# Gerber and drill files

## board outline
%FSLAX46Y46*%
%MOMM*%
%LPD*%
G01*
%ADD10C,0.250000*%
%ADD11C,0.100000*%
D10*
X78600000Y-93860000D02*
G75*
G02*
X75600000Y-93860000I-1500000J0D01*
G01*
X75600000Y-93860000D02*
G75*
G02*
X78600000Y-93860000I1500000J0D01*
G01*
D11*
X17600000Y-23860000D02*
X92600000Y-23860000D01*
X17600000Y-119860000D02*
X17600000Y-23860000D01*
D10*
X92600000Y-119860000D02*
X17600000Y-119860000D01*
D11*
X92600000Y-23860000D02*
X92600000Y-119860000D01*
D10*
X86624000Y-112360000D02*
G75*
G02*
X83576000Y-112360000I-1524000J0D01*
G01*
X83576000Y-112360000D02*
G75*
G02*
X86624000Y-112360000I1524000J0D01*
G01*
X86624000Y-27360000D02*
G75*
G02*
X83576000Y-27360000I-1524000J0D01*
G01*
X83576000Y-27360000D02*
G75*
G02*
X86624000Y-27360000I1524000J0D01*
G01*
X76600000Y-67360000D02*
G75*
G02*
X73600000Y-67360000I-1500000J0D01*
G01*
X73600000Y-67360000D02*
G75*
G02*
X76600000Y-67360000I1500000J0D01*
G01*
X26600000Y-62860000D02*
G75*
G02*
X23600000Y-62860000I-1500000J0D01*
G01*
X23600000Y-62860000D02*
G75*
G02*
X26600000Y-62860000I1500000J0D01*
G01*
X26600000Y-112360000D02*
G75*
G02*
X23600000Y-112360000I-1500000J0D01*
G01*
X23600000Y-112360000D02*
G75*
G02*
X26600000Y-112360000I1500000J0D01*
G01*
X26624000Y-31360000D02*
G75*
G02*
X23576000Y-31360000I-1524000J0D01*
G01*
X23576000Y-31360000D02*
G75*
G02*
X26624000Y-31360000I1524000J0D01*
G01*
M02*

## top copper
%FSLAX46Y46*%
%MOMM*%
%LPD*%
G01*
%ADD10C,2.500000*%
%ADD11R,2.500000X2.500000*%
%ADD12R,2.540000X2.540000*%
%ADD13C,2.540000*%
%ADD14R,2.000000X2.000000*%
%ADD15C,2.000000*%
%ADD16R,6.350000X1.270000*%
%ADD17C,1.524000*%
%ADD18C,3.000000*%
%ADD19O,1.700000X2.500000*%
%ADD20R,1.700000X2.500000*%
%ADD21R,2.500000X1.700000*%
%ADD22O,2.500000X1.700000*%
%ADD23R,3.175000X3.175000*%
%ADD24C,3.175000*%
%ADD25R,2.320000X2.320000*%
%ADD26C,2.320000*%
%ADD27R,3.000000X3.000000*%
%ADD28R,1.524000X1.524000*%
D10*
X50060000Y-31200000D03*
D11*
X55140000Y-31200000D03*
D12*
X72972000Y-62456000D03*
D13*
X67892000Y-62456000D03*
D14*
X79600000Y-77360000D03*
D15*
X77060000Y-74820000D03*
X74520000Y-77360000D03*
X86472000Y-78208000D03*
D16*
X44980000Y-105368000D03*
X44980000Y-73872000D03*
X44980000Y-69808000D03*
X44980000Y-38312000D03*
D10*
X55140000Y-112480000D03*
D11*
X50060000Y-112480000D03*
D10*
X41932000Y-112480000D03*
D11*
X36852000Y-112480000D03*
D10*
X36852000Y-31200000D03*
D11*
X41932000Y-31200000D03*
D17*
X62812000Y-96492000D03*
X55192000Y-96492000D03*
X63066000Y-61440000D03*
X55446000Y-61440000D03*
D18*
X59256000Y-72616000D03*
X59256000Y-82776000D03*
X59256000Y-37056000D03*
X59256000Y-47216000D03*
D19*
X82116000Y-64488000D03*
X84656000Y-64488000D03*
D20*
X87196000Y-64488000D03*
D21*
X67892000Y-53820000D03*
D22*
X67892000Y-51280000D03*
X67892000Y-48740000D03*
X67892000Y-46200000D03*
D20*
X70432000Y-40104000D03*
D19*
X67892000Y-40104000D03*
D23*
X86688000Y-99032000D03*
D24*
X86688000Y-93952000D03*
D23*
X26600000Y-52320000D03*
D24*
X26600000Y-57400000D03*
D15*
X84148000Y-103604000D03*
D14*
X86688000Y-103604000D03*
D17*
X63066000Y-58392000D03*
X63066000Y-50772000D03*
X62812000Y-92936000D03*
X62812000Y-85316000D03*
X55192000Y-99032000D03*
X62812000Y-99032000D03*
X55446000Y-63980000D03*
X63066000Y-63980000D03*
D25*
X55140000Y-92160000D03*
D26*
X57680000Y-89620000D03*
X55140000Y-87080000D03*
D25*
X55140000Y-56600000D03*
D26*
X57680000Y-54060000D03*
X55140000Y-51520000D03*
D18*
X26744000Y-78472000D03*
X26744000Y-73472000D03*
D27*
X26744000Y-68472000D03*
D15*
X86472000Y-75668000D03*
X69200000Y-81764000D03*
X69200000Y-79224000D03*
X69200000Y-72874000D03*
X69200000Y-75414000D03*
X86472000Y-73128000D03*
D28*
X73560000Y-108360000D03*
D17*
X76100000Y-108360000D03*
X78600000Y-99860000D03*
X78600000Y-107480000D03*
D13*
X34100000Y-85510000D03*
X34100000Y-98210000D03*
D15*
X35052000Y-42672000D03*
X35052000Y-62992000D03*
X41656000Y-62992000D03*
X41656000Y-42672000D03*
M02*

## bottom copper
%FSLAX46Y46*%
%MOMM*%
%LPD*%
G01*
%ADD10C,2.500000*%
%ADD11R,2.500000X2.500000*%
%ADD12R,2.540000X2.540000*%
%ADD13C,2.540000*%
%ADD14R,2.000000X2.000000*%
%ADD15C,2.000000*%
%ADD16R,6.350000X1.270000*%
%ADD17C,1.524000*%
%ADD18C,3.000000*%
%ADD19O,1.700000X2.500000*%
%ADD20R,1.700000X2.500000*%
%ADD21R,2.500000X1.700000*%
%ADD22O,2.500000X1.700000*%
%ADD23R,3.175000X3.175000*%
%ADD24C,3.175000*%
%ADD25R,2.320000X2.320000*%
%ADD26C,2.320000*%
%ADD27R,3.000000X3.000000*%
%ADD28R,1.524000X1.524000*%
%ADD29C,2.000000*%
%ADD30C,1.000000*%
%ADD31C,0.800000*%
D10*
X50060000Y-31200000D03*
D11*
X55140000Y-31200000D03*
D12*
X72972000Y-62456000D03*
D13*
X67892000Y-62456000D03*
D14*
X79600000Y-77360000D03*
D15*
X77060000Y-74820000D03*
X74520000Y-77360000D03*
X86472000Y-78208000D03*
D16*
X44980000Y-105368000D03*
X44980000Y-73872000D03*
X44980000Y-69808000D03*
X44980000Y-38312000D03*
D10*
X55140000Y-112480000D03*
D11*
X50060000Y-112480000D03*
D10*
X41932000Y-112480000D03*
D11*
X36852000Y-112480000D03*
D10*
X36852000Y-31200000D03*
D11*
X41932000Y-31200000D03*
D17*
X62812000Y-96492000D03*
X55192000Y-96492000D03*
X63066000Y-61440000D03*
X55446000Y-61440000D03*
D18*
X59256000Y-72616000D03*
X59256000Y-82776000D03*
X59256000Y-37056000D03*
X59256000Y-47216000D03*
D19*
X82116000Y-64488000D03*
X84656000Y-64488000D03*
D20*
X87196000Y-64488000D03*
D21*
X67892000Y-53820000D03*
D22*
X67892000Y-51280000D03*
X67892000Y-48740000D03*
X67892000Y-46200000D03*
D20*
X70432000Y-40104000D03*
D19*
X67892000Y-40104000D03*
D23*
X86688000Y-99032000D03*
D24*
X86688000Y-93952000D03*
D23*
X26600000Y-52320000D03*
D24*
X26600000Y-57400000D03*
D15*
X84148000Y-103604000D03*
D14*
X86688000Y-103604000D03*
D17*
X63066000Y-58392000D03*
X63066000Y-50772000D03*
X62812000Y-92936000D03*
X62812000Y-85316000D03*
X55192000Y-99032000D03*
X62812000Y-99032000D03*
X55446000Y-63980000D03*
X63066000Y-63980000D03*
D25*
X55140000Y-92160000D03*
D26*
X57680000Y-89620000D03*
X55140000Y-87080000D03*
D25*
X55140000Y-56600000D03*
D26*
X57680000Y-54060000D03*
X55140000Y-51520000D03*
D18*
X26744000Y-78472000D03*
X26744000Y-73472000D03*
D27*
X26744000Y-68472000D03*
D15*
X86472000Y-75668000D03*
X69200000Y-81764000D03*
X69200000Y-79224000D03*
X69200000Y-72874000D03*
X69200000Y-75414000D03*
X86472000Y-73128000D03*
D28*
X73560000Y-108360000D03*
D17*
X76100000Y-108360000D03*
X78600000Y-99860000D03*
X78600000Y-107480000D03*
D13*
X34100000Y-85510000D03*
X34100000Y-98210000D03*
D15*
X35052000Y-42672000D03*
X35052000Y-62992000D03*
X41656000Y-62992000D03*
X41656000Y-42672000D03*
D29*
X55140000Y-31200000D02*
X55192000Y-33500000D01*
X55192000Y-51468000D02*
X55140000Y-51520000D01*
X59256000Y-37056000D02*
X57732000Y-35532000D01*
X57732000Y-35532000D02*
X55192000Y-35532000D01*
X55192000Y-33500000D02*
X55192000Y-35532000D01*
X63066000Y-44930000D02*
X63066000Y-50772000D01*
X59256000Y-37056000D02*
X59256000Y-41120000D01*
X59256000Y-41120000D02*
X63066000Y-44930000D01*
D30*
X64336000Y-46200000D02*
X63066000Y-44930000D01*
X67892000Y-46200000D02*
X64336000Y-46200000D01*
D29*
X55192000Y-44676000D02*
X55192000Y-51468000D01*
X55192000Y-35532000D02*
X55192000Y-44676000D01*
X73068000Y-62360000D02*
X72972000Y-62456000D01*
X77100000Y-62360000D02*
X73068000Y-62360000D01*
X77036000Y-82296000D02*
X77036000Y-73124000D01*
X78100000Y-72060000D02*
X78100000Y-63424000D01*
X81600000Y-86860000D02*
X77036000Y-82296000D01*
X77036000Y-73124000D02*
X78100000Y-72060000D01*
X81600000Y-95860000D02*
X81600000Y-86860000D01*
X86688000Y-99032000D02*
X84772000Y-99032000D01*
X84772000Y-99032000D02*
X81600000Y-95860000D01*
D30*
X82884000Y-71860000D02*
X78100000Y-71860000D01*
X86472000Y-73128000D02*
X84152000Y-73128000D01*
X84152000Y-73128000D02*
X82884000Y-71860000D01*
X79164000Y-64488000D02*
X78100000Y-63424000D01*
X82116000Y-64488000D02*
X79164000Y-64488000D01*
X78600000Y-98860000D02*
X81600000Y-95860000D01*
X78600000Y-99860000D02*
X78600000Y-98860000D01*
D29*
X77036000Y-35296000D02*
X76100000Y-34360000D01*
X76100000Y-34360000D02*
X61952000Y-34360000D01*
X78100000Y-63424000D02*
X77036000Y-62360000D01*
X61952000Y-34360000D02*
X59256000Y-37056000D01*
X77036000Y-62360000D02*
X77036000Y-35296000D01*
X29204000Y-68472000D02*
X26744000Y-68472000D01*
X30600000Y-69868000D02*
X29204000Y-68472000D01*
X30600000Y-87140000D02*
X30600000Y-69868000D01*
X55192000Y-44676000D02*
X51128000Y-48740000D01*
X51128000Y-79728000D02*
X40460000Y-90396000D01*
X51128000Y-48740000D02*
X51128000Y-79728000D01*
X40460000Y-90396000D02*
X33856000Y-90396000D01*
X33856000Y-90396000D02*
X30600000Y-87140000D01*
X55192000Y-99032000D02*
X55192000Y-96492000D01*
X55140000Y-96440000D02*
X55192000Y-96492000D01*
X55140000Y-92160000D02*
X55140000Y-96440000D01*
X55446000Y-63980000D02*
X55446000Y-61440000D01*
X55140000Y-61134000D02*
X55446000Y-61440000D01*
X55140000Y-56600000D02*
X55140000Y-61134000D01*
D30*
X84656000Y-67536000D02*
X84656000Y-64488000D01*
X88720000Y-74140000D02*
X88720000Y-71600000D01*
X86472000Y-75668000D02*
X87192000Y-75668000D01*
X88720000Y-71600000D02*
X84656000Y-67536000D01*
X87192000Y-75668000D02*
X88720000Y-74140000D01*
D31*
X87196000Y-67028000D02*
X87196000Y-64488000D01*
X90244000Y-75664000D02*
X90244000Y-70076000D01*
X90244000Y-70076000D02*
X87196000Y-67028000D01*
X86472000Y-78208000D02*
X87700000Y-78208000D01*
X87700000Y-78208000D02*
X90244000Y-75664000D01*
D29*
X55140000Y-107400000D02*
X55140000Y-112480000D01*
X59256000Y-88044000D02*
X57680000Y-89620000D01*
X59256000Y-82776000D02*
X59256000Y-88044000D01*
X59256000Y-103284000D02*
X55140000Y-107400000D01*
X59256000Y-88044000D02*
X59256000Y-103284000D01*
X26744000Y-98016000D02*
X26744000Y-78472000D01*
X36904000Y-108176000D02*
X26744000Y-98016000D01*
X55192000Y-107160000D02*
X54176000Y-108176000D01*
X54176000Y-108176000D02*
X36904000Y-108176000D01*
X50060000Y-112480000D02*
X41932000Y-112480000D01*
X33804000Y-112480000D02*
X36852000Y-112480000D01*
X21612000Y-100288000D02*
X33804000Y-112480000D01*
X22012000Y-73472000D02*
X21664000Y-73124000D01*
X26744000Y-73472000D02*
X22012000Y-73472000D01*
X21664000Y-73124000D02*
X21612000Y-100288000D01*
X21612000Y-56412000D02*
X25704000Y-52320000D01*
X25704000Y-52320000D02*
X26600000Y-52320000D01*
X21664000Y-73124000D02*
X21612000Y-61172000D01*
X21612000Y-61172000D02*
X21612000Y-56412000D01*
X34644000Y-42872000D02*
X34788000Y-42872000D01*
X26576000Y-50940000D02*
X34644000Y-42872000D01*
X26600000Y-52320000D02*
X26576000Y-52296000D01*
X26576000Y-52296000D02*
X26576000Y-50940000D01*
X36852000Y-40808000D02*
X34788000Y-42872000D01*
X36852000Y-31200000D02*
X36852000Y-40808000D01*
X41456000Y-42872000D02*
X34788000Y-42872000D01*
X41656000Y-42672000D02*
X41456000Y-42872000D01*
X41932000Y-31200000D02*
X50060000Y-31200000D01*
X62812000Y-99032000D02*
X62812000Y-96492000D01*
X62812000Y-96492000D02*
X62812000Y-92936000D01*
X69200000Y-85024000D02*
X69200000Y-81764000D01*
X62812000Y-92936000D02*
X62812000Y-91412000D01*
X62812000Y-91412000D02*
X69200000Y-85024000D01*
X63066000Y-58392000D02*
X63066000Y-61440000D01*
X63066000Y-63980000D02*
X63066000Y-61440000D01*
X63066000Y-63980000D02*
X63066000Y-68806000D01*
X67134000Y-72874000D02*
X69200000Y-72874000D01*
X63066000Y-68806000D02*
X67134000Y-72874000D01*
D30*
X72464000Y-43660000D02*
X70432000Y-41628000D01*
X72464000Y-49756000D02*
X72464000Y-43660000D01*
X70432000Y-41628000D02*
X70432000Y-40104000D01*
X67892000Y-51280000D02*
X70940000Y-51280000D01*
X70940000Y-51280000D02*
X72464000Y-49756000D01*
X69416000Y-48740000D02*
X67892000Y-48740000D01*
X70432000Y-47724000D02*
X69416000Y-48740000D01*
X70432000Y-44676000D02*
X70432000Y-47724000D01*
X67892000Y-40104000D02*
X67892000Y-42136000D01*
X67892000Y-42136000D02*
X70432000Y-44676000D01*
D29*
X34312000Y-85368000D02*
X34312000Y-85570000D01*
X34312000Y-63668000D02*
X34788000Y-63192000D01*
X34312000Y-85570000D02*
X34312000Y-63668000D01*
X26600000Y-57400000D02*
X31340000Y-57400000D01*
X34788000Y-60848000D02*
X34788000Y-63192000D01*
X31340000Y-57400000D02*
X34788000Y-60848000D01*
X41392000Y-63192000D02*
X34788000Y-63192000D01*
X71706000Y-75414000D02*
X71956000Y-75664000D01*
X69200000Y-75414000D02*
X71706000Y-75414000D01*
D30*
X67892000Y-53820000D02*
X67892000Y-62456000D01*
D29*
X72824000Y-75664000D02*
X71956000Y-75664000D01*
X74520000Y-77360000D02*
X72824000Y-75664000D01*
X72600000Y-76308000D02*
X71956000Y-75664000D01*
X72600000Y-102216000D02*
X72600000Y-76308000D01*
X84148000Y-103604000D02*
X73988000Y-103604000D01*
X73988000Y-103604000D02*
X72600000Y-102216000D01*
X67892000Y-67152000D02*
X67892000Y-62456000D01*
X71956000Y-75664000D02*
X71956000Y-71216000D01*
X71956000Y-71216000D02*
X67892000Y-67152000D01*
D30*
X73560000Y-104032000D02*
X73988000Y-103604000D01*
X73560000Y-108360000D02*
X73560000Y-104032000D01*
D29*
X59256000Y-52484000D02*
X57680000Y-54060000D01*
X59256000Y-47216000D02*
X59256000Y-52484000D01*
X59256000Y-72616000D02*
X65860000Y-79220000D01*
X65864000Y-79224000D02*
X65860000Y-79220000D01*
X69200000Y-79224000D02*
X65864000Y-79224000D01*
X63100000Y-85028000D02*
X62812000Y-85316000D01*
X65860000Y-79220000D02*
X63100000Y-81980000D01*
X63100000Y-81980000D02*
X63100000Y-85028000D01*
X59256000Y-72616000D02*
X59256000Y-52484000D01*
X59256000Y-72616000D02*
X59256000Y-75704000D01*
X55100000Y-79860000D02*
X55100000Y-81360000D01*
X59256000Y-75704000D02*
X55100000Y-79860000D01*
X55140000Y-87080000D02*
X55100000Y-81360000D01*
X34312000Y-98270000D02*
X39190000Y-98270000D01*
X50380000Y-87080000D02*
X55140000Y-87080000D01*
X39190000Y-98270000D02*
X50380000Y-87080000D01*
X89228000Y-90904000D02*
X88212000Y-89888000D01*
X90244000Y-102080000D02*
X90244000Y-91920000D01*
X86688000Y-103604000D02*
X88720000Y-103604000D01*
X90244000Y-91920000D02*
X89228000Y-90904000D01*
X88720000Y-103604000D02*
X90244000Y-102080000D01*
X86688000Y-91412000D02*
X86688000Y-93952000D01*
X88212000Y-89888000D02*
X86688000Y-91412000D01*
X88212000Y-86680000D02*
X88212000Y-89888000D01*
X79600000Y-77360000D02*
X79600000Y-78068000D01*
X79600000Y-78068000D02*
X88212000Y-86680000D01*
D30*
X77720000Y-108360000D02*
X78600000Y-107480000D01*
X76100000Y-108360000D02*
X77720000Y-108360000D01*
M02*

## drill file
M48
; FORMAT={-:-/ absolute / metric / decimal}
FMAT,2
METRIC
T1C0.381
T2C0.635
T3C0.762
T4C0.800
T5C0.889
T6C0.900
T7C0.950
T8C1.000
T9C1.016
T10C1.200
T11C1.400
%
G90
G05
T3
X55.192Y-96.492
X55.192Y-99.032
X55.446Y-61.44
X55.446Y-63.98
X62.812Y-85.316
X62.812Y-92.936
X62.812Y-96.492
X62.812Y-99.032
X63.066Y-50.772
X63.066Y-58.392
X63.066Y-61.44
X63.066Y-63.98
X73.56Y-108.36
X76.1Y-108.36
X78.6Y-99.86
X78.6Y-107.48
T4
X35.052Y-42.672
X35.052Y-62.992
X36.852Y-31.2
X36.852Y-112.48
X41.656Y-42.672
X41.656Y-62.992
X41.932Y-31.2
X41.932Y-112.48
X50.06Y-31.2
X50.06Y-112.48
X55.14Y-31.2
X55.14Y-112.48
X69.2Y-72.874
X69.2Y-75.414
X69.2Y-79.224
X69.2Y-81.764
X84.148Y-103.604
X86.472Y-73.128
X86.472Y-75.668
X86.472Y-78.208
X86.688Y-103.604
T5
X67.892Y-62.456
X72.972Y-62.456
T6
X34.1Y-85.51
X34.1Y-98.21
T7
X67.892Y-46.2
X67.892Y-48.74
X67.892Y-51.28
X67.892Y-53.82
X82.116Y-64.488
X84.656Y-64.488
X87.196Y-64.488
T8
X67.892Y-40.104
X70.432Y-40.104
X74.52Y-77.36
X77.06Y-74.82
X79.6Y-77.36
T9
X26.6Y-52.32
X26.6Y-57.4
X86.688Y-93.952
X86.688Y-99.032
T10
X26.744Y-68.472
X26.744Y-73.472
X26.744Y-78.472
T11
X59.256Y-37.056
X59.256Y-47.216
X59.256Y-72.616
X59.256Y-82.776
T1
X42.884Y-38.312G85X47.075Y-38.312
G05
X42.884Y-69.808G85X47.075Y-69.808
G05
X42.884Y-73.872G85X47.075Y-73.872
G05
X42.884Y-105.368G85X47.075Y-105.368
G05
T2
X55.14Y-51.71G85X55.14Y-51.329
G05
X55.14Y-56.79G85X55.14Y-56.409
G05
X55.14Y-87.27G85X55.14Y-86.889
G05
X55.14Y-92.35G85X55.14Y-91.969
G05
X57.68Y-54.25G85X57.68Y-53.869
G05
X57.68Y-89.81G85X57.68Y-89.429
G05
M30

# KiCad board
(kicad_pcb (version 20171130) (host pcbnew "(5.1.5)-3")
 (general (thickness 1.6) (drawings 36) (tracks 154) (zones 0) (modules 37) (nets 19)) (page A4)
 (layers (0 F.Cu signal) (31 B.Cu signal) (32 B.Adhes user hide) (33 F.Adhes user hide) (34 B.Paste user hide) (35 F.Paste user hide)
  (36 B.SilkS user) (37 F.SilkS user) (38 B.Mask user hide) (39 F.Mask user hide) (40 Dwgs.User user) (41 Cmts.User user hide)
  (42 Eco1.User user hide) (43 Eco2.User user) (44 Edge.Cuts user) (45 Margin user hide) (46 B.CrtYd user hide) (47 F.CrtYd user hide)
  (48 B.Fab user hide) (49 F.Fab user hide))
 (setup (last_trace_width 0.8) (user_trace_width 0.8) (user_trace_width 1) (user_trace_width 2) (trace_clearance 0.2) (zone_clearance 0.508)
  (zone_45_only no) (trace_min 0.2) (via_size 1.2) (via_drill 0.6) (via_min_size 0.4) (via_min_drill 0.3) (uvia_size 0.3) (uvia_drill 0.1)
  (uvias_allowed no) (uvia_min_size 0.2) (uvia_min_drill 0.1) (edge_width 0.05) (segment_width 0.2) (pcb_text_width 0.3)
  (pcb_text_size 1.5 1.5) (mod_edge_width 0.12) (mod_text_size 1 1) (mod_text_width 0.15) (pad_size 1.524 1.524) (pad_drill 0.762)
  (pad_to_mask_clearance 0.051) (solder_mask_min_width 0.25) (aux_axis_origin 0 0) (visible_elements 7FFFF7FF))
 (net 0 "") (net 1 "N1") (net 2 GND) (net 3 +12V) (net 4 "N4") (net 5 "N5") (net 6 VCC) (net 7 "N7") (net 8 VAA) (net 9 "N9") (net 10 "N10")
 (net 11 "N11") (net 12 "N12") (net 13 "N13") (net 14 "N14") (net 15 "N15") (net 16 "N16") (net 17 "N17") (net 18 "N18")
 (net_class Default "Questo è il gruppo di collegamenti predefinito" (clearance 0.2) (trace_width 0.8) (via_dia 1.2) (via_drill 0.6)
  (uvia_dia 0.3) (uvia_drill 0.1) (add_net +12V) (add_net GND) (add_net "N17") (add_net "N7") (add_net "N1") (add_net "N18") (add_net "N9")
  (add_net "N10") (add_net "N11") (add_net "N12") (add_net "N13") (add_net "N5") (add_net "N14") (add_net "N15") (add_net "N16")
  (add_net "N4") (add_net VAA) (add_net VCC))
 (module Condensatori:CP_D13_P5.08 (layer F.Cu) (at 52.6 31.2 180)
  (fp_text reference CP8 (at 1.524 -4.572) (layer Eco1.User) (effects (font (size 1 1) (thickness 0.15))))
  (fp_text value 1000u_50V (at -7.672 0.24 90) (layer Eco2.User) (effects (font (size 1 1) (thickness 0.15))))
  (pad 2 thru_hole circle (at 2.54 0 180) (size 2.5 2.5) (drill 0.8) (layers *.Cu *.Mask) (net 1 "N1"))
  (pad 1 thru_hole rect (at -2.54 0 180) (size 2.5 2.5) (drill 0.8) (layers *.Cu *.Mask) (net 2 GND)))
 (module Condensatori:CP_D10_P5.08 (layer F.Cu) (at 72.972 62.456 180)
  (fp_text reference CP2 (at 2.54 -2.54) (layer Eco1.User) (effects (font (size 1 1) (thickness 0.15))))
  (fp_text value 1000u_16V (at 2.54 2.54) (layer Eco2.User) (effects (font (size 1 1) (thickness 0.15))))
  (pad 1 thru_hole rect (at 0 0 180) (size 2.54 2.54) (drill 0.889) (layers *.Cu *.Mask) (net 2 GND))
  (pad 2 thru_hole circle (at 5.08 0 180) (size 2.54 2.54) (drill 0.889) (layers *.Cu *.Mask) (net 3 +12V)))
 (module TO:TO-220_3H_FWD (layer F.Cu) (at 79.6 77.36 180)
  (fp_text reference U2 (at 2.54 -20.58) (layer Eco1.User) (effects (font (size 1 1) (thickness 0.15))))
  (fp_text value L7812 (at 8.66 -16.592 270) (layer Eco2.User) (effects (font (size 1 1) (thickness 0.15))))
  (pad 1 thru_hole rect (at 0 0 180) (size 2 2) (drill 1) (layers *.Cu *.Mask) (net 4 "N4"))
  (pad 2 thru_hole circle (at 2.54 2.54 180) (size 2 2) (drill 1) (layers *.Cu *.Mask) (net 2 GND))
  (pad 3 thru_hole circle (at 5.08 0 180) (size 2 2) (drill 1) (layers *.Cu *.Mask) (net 3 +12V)))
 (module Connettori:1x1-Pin (layer F.Cu) (at 86.472 78.208 180)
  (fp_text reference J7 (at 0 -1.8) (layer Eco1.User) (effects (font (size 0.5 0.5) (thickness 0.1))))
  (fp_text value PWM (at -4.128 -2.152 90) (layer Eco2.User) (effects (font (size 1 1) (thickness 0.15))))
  (pad 1 thru_hole circle (at 0 0 180) (size 2 2) (drill 0.8) (layers *.Cu *.Mask) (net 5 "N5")))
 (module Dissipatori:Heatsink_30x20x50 (layer F.Cu) (at 32.28 104.86 90)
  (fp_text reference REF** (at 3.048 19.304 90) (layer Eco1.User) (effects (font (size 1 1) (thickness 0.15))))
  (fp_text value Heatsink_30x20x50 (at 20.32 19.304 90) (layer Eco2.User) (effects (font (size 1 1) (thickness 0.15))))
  (pad "" thru_hole rect (at -0.508 12.7 90) (size 1.27 6.35) (drill oval 0.381 4.572) (layers *.Cu *.Mask))
  (pad "" thru_hole rect (at 30.988 12.7 90) (size 1.27 6.35) (drill oval 0.381 4.572) (layers *.Cu *.Mask)))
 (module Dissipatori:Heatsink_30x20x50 (layer F.Cu) (at 32.28 69.3 90)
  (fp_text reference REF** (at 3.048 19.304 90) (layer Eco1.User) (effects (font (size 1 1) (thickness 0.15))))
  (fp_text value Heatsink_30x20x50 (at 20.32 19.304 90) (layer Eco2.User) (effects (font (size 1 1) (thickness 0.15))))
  (pad "" thru_hole rect (at -0.508 12.7 90) (size 1.27 6.35) (drill oval 0.381 4.572) (layers *.Cu *.Mask))
  (pad "" thru_hole rect (at 30.988 12.7 90) (size 1.27 6.35) (drill oval 0.381 4.572) (layers *.Cu *.Mask)))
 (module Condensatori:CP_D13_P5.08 (layer F.Cu) (at 52.6 112.48)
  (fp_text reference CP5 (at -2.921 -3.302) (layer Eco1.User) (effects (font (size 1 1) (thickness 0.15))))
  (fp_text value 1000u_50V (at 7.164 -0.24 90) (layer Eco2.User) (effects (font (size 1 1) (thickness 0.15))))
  (pad 2 thru_hole circle (at 2.54 0) (size 2.5 2.5) (drill 0.8) (layers *.Cu *.Mask) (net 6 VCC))
  (pad 1 thru_hole rect (at -2.54 0) (size 2.5 2.5) (drill 0.8) (layers *.Cu *.Mask) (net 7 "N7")))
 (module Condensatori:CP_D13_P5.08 (layer F.Cu) (at 39.392 112.48)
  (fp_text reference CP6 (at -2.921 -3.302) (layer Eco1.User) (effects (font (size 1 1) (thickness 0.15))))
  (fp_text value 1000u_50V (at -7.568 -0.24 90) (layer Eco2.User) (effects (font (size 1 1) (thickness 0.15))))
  (pad 2 thru_hole circle (at 2.54 0) (size 2.5 2.5) (drill 0.8) (layers *.Cu *.Mask) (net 7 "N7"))
  (pad 1 thru_hole rect (at -2.54 0) (size 2.5 2.5) (drill 0.8) (layers *.Cu *.Mask) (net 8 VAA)))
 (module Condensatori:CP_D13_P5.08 (layer F.Cu) (at 39.392 31.2 180)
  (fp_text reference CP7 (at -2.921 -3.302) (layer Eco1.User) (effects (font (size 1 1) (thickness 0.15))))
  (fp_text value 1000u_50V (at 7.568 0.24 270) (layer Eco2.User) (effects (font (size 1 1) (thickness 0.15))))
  (pad 2 thru_hole circle (at 2.54 0 180) (size 2.5 2.5) (drill 0.8) (layers *.Cu *.Mask) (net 8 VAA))
  (pad 1 thru_hole rect (at -2.54 0 180) (size 2.5 2.5) (drill 0.8) (layers *.Cu *.Mask) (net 1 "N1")))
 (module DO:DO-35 (layer F.Cu) (at 59.002 96.492 180)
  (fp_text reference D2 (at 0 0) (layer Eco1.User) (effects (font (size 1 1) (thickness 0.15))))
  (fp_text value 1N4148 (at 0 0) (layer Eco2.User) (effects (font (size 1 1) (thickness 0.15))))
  (pad 1 thru_hole circle (at -3.81 0 180) (size 1.524 1.524) (drill 0.762) (layers *.Cu *.Mask) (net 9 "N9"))
  (pad 2 thru_hole circle (at 3.81 0 180) (size 1.524 1.524) (drill 0.762) (layers *.Cu *.Mask) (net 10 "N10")))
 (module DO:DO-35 (layer F.Cu) (at 59.256 61.44 180)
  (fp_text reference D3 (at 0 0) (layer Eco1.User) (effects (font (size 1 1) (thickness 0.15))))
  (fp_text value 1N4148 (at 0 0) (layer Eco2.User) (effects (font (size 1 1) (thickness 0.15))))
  (pad 1 thru_hole circle (at -3.81 0 180) (size 1.524 1.524) (drill 0.762) (layers *.Cu *.Mask) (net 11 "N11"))
  (pad 2 thru_hole circle (at 3.81 0 180) (size 1.524 1.524) (drill 0.762) (layers *.Cu *.Mask) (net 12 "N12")))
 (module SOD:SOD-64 (layer F.Cu) (at 59.256 77.696 90)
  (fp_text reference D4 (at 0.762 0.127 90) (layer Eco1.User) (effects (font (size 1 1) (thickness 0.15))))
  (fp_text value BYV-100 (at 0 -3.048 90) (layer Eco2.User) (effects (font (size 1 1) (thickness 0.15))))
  (pad 2 thru_hole circle (at 5.08 0 90) (size 3 3) (drill 1.4) (layers *.Cu *.Mask) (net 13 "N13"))
  (pad 1 thru_hole circle (at -5.08 0 90) (size 3 3) (drill 1.4) (layers *.Cu *.Mask) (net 6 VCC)))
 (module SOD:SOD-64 (layer F.Cu) (at 59.256 42.136 90)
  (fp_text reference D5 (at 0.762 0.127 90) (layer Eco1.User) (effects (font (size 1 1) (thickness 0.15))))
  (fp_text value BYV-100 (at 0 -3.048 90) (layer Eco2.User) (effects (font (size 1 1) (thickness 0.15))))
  (pad 2 thru_hole circle (at 5.08 0 90) (size 3 3) (drill 1.4) (layers *.Cu *.Mask) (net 2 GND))
  (pad 1 thru_hole circle (at -5.08 0 90) (size 3 3) (drill 1.4) (layers *.Cu *.Mask) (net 13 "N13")))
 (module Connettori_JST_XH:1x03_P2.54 (layer F.Cu) (at 87.196 64.488 180)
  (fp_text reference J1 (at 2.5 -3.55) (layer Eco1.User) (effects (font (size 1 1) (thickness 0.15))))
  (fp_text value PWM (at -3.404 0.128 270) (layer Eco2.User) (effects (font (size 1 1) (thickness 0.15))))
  (pad 3 thru_hole oval (at 5.08 0 180) (size 1.7 2.5) (drill 0.95) (layers *.Cu *.Mask) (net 2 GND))
  (pad 2 thru_hole oval (at 2.54 0 180) (size 1.7 2.5) (drill 0.95) (layers *.Cu *.Mask) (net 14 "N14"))
  (pad 1 thru_hole rect (at 0 0 180) (size 1.7 2.5) (drill 0.95) (layers *.Cu *.Mask) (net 5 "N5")))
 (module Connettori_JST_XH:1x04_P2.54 (layer F.Cu) (at 67.892 53.82 90)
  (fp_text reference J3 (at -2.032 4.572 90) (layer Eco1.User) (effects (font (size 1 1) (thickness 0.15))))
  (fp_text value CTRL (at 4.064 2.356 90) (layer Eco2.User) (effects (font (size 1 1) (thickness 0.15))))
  (pad 1 thru_hole rect (at 0 0 90) (size 1.7 2.5) (drill 0.95) (layers *.Cu *.Mask) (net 3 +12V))
  (pad 2 thru_hole oval (at 2.54 0 90) (size 1.7 2.5) (drill 0.95) (layers *.Cu *.Mask) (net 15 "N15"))
  (pad 3 thru_hole oval (at 5.08 0 90) (size 1.7 2.5) (drill 0.95) (layers *.Cu *.Mask) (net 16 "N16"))
  (pad 4 thru_hole oval (at 7.62 0 90) (size 1.7 2.5) (drill 0.95) (layers *.Cu *.Mask) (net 2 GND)))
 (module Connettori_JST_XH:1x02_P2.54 (layer F.Cu) (at 70.432 40.104 180)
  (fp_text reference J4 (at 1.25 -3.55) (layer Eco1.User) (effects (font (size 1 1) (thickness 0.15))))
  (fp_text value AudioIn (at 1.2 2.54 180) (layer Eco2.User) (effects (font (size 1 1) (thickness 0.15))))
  (pad 1 thru_hole rect (at 0 0 180) (size 1.7 2.5) (drill 1) (layers *.Cu *.Mask) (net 15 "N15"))
  (pad 2 thru_hole oval (at 2.54 0 180) (size 1.7 2.5) (drill 1) (layers *.Cu *.Mask) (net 16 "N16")))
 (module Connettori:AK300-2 (layer F.Cu) (at 86.688 96.492 90)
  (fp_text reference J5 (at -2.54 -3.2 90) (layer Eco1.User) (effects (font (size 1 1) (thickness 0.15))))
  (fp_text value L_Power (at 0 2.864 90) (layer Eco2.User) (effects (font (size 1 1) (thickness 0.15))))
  (pad 1 thru_hole rect (at -2.54 0 90) (size 3.175 3.175) (drill 1.016) (layers *.Cu F.Paste F.Mask) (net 2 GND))
  (pad 2 thru_hole circle (at 2.54 0 90) (size 3.175 3.175) (drill 1.016) (layers *.Cu F.Paste F.Mask) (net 4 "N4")))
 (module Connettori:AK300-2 (layer F.Cu) (at 26.6 54.86 270)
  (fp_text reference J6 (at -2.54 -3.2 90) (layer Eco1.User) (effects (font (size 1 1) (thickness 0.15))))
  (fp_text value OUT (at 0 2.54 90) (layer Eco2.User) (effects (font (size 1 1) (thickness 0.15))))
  (pad 1 thru_hole rect (at -2.54 0 270) (size 3.175 3.175) (drill 1.016) (layers *.Cu F.Paste F.Mask) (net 8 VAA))
  (pad 2 thru_hole circle (at 2.54 0 270) (size 3.175 3.175) (drill 1.016) (layers *.Cu F.Paste F.Mask) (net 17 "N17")))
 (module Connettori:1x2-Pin (layer F.Cu) (at 86.688 103.604 270)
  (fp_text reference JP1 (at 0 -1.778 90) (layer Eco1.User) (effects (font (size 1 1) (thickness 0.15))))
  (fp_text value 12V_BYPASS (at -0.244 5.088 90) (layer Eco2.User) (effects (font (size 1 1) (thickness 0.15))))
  (pad 2 thru_hole circle (at 0 2.54 180) (size 2 2) (drill 0.8) (layers *.Cu *.Mask) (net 3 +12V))
  (pad 1 thru_hole rect (at 0 0 180) (size 2 2) (drill 0.8) (layers *.Cu *.Mask) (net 4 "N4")))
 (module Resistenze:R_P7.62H (layer F.Cu) (at 63.066 54.582 270)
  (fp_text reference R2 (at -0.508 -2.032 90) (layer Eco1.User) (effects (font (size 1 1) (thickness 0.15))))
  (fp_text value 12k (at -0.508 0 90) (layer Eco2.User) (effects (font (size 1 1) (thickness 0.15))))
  (pad 2 thru_hole circle (at 3.81 0 270) (size 1.524 1.524) (drill 0.762) (layers *.Cu *.Mask) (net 11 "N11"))
  (pad 1 thru_hole circle (at -3.81 0 270) (size 1.524 1.524) (drill 0.762) (layers *.Cu *.Mask) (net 2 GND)))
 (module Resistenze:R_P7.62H (layer F.Cu) (at 62.812 89.126 270)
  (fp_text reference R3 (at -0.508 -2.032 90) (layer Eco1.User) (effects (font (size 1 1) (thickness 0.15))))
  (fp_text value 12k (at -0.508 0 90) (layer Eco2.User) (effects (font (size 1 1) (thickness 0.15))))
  (pad 2 thru_hole circle (at 3.81 0 270) (size 1.524 1.524) (drill 0.762) (layers *.Cu *.Mask) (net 9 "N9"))
  (pad 1 thru_hole circle (at -3.81 0 270) (size 1.524 1.524) (drill 0.762) (layers *.Cu *.Mask) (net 13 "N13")))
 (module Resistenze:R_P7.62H (layer F.Cu) (at 59.002 99.032 180)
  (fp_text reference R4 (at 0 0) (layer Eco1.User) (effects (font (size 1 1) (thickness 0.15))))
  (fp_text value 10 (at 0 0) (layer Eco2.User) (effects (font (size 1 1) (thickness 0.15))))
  (pad 2 thru_hole circle (at 3.81 0 180) (size 1.524 1.524) (drill 0.762) (layers *.Cu *.Mask) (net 10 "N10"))
  (pad 1 thru_hole circle (at -3.81 0 180) (size 1.524 1.524) (drill 0.762) (layers *.Cu *.Mask) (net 9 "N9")))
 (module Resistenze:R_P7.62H (layer F.Cu) (at 59.256 63.98 180)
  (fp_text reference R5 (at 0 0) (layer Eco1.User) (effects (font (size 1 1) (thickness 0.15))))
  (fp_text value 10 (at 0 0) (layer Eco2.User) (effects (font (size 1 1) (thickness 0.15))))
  (pad 2 thru_hole circle (at 3.81 0 180) (size 1.524 1.524) (drill 0.762) (layers *.Cu *.Mask) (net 12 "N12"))
  (pad 1 thru_hole circle (at -3.81 0 180) (size 1.524 1.524) (drill 0.762) (layers *.Cu *.Mask) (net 11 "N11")))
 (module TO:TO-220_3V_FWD (layer F.Cu) (at 55.14 89.62 90)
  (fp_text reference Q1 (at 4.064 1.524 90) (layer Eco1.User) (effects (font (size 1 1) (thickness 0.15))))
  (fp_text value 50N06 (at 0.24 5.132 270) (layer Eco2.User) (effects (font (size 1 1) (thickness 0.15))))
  (pad 1 thru_hole rect (at -2.54 0 90) (size 2.32 2.32) (drill oval 1.016 0.635) (layers *.Cu *.Mask) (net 10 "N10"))
  (pad 2 thru_hole circle (at 0 2.54 90) (size 2.32 2.32) (drill oval 1.016 0.635) (layers *.Cu *.Mask) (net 6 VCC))
  (pad 3 thru_hole circle (at 2.54 0 90) (size 2.32 2.32) (drill oval 1.016 0.635) (layers *.Cu *.Mask) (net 13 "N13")))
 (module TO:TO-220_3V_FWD (layer F.Cu) (at 55.14 54.06 90)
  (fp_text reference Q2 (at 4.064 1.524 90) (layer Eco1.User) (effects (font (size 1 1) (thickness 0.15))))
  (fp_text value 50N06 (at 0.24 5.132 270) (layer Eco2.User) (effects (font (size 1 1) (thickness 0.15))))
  (pad 1 thru_hole rect (at -2.54 0 90) (size 2.32 2.32) (drill oval 1.016 0.635) (layers *.Cu *.Mask) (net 12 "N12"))
  (pad 2 thru_hole circle (at 0 2.54 90) (size 2.32 2.32) (drill oval 1.016 0.635) (layers *.Cu *.Mask) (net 13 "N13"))
  (pad 3 thru_hole circle (at 2.54 0 90) (size 2.32 2.32) (drill oval 1.016 0.635) (layers *.Cu *.Mask) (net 2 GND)))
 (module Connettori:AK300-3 (layer F.Cu) (at 26.744 73.552 270)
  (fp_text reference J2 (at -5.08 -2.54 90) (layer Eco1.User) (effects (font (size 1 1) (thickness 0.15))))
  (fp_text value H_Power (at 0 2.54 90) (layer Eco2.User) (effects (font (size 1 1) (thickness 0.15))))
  (pad 3 thru_hole circle (at 4.92 0 270) (size 3 3) (drill 1.2) (layers *.Cu F.Paste F.Mask) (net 6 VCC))
  (pad 2 thru_hole circle (at -0.08 0 270) (size 3 3) (drill 1.2) (layers *.Cu F.Paste F.Mask) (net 8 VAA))
  (pad 1 thru_hole rect (at -5.08 0 270) (size 3 3) (drill 1.2) (layers *.Cu F.Paste F.Mask) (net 2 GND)))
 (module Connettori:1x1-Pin (layer F.Cu) (at 86.472 75.668 180)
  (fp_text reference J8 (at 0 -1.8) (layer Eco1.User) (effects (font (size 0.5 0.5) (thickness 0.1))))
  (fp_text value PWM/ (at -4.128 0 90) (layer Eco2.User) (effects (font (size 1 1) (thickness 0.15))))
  (pad 1 thru_hole circle (at 0 0 180) (size 2 2) (drill 0.8) (layers *.Cu *.Mask) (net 14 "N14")))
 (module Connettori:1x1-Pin (layer F.Cu) (at 69.2 81.764)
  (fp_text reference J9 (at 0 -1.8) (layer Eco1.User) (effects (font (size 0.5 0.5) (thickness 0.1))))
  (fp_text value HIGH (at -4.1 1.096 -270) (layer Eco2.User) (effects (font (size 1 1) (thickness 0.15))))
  (pad 1 thru_hole circle (at 0 0) (size 2 2) (drill 0.8) (layers *.Cu *.Mask) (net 9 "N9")))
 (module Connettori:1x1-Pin (layer F.Cu) (at 69.2 79.224)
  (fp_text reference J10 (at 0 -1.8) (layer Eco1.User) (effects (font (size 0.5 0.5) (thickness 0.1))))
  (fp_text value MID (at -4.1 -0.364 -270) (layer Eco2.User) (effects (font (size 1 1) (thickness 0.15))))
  (pad 1 thru_hole circle (at 0 0) (size 2 2) (drill 0.8) (layers *.Cu *.Mask) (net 13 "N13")))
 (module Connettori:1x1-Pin (layer F.Cu) (at 69.2 72.874)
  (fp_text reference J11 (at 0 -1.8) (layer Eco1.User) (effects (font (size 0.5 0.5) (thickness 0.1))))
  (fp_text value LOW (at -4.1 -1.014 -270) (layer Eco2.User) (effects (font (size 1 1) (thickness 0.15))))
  (pad 1 thru_hole circle (at 0 0) (size 2 2) (drill 0.8) (layers *.Cu *.Mask) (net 11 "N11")))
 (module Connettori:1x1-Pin (layer F.Cu) (at 69.2 75.414)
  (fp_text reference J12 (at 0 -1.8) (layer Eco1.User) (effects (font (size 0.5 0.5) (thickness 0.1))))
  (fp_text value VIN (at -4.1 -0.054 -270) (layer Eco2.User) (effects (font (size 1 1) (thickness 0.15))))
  (pad 1 thru_hole circle (at 0 0) (size 2 2) (drill 0.8) (layers *.Cu *.Mask) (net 3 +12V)))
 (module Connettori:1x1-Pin (layer F.Cu) (at 86.472 73.128 180)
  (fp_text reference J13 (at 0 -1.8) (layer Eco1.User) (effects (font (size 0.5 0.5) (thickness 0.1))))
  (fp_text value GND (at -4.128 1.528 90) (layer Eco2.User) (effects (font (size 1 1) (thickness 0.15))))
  (pad 1 thru_hole circle (at 0 0 180) (size 2 2) (drill 0.8) (layers *.Cu *.Mask) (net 2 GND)))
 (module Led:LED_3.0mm (layer F.Cu) (at 73.56 108.36)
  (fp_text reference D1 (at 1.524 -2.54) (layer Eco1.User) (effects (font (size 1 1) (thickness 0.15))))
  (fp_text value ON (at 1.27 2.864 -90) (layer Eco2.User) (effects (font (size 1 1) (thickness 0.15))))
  (pad 1 thru_hole rect (at 0 0) (size 1.524 1.524) (drill 0.762) (layers *.Cu *.Mask) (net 3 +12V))
  (pad 2 thru_hole circle (at 2.54 0) (size 1.524 1.524) (drill 0.762) (layers *.Cu *.Mask) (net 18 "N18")))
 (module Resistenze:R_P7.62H (layer F.Cu) (at 78.6 103.67 90)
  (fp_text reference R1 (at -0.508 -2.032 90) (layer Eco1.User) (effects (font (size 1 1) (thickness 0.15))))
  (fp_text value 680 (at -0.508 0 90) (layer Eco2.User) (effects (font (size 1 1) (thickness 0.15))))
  (pad 2 thru_hole circle (at 3.81 0 90) (size 1.524 1.524) (drill 0.762) (layers *.Cu *.Mask) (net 2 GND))
  (pad 1 thru_hole circle (at -3.81 0 90) (size 1.524 1.524) (drill 0.762) (layers *.Cu *.Mask) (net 18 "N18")))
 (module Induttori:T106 (layer F.Cu) (at 34.1 91.86 90)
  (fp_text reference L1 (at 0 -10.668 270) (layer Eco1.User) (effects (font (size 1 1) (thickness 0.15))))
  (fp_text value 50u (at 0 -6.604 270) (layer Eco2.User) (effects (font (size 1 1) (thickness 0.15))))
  (pad 2 thru_hole circle (at 6.35 0 90) (size 2.54 2.54) (drill 0.9) (layers *.Cu *.Mask) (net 17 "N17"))
  (pad 1 thru_hole circle (at -6.35 0 90) (size 2.54 2.54) (drill 0.9) (layers *.Cu *.Mask) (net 13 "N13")))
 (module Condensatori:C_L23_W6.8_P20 (layer F.Cu) (at 35.052 42.672 270)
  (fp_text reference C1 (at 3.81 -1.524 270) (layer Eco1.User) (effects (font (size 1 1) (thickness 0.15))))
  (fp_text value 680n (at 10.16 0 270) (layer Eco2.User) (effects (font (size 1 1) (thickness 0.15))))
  (pad 1 thru_hole circle (at 0 0 270) (size 2 2) (drill 0.8) (layers *.Cu *.Mask) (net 8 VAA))
  (pad 2 thru_hole circle (at 20.32 0 270) (size 2 2) (drill 0.8) (layers *.Cu *.Mask) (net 17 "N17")))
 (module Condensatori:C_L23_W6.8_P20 (layer F.Cu) (at 41.656 42.672 270)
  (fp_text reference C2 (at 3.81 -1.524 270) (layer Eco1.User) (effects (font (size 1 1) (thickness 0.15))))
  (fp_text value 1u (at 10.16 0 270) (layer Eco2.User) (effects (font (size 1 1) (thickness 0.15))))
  (pad 2 thru_hole circle (at 20.32 0 270) (size 2 2) (drill 0.8) (layers *.Cu *.Mask) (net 17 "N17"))
  (pad 1 thru_hole circle (at 0 0 270) (size 2 2) (drill 0.8) (layers *.Cu *.Mask) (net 8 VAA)))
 (gr_circle (center 77.1 93.86) (end 77.1 92.36) (layer Edge.Cuts) (width 0.25))
 (gr_line (start 17.6 23.86) (end 92.6 23.86) (layer Edge.Cuts) (width 0.1))
 (gr_line (start 17.6 119.86) (end 17.6 23.86) (layer Edge.Cuts) (width 0.1))
 (gr_line (start 92.6 119.86) (end 17.6 119.86) (layer Edge.Cuts) (width 0.25))
 (gr_line (start 92.6 23.86) (end 92.6 119.86) (layer Edge.Cuts) (width 0.1))
 (gr_circle (center 85.1 112.36) (end 85.1 110.836) (layer Edge.Cuts) (width 0.25))
 (gr_circle (center 85.1 27.36) (end 85.1 25.836) (layer Edge.Cuts) (width 0.25))
 (gr_circle (center 75.1 67.36) (end 75.1 65.86) (layer Edge.Cuts) (width 0.25))
 (gr_circle (center 25.1 62.86) (end 25.1 61.36) (layer Edge.Cuts) (width 0.25))
 (gr_circle (center 25.1 112.36) (end 25.1 110.86) (layer Edge.Cuts) (width 0.25))
 (gr_circle (center 25.1 31.36) (end 25.1 29.836) (layer Edge.Cuts) (width 0.25))
 (segment (start 55.14 31.2) (end 55.192 33.5) (width 2) (layer B.Cu) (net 2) (status 10))
 (segment (start 55.192 51.468) (end 55.14 51.52) (width 2) (layer B.Cu) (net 2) (status 30))
 (segment (start 59.256 37.056) (end 57.732 35.532) (width 2) (layer B.Cu) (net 2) (status 10))
 (segment (start 57.732 35.532) (end 55.192 35.532) (width 2) (layer B.Cu) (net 2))
 (segment (start 55.192 33.5) (end 55.192 35.532) (width 2) (layer B.Cu) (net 2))
 (segment (start 63.066 44.93) (end 63.066 50.772) (width 2) (layer B.Cu) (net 2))
 (segment (start 59.256 37.056) (end 59.256 41.12) (width 2) (layer B.Cu) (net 2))
 (segment (start 59.256 41.12) (end 63.066 44.93) (width 2) (layer B.Cu) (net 2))
 (segment (start 64.336 46.2) (end 63.066 44.93) (width 1) (layer B.Cu) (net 2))
 (segment (start 67.892 46.2) (end 64.336 46.2) (width 1) (layer B.Cu) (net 2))
 (segment (start 55.192 44.676) (end 55.192 51.468) (width 2) (layer B.Cu) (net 2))
 (segment (start 55.192 35.532) (end 55.192 44.676) (width 2) (layer B.Cu) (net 2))
 (segment (start 73.068 62.36) (end 72.972 62.456) (width 2) (layer B.Cu) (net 2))
 (segment (start 77.1 62.36) (end 73.068 62.36) (width 2) (layer B.Cu) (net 2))
 (segment (start 77.036 82.296) (end 77.036 73.124) (width 2) (layer B.Cu) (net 2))
 (segment (start 78.1 72.06) (end 78.1 63.424) (width 2) (layer B.Cu) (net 2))
 (segment (start 81.6 86.86) (end 77.036 82.296) (width 2) (layer B.Cu) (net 2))
 (segment (start 77.036 73.124) (end 78.1 72.06) (width 2) (layer B.Cu) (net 2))
 (segment (start 81.6 95.86) (end 81.6 86.86) (width 2) (layer B.Cu) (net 2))
 (segment (start 86.688 99.032) (end 84.772 99.032) (width 2) (layer B.Cu) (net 2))
 (segment (start 84.772 99.032) (end 81.6 95.86) (width 2) (layer B.Cu) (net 2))
 (segment (start 82.884 71.86) (end 78.1 71.86) (width 1) (layer B.Cu) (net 2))
 (segment (start 86.472 73.128) (end 84.152 73.128) (width 1) (layer B.Cu) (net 2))
 (segment (start 84.152 73.128) (end 82.884 71.86) (width 1) (layer B.Cu) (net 2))
 (segment (start 79.164 64.488) (end 78.1 63.424) (width 1) (layer B.Cu) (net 2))
 (segment (start 82.116 64.488) (end 79.164 64.488) (width 1) (layer B.Cu) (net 2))
 (segment (start 78.6 98.86) (end 81.6 95.86) (width 1) (layer B.Cu) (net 2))
 (segment (start 78.6 99.86) (end 78.6 98.86) (width 1) (layer B.Cu) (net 2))
 (segment (start 77.036 35.296) (end 76.1 34.36) (width 2) (layer B.Cu) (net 2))
 (segment (start 76.1 34.36) (end 61.952 34.36) (width 2) (layer B.Cu) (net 2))
 (segment (start 78.1 63.424) (end 77.036 62.36) (width 2) (layer B.Cu) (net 2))
 (segment (start 61.952 34.36) (end 59.256 37.056) (width 2) (layer B.Cu) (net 2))
 (segment (start 77.036 62.36) (end 77.036 35.296) (width 2) (layer B.Cu) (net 2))
 (segment (start 29.204 68.472) (end 26.744 68.472) (width 2) (layer B.Cu) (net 2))
 (segment (start 30.6 69.868) (end 29.204 68.472) (width 2) (layer B.Cu) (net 2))
 (segment (start 30.6 87.14) (end 30.6 69.868) (width 2) (layer B.Cu) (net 2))
 (segment (start 55.192 44.676) (end 51.128 48.74) (width 2) (layer B.Cu) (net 2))
 (segment (start 51.128 79.728) (end 40.46 90.396) (width 2) (layer B.Cu) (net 2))
 (segment (start 51.128 48.74) (end 51.128 79.728) (width 2) (layer B.Cu) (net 2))
 (segment (start 40.46 90.396) (end 33.856 90.396) (width 2) (layer B.Cu) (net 2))
 (segment (start 33.856 90.396) (end 30.6 87.14) (width 2) (layer B.Cu) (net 2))
 (segment (start 55.192 99.032) (end 55.192 96.492) (width 2) (layer B.Cu) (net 10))
 (segment (start 55.14 96.44) (end 55.192 96.492) (width 2) (layer B.Cu) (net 10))
 (segment (start 55.14 92.16) (end 55.14 96.44) (width 2) (layer B.Cu) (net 10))
 (segment (start 55.446 63.98) (end 55.446 61.44) (width 2) (layer B.Cu) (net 12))
 (segment (start 55.14 61.134) (end 55.446 61.44) (width 2) (layer B.Cu) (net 12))
 (segment (start 55.14 56.6) (end 55.14 61.134) (width 2) (layer B.Cu) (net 12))
 (segment (start 84.656 67.536) (end 84.656 64.488) (width 1) (layer B.Cu) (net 14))
 (segment (start 88.72 74.14) (end 88.72 71.6) (width 1) (layer B.Cu) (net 14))
 (segment (start 86.472 75.668) (end 87.192 75.668) (width 1) (layer B.Cu) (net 14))
 (segment (start 88.72 71.6) (end 84.656 67.536) (width 1) (layer B.Cu) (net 14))
 (segment (start 87.192 75.668) (end 88.72 74.14) (width 1) (layer B.Cu) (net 14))
 (segment (start 87.196 67.028) (end 87.196 64.488) (width 0.8) (layer B.Cu) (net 5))
 (segment (start 90.244 75.664) (end 90.244 70.076) (width 0.8) (layer B.Cu) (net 5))
 (segment (start 90.244 70.076) (end 87.196 67.028) (width 0.8) (layer B.Cu) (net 5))
 (segment (start 86.472 78.208) (end 87.7 78.208) (width 0.8) (layer B.Cu) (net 5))
 (segment (start 87.7 78.208) (end 90.244 75.664) (width 0.8) (layer B.Cu) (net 5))
 (segment (start 55.14 107.4) (end 55.14 112.48) (width 2) (layer B.Cu) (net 6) (status 20))
 (segment (start 59.256 88.044) (end 57.68 89.62) (width 2) (layer B.Cu) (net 6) (status 20))
 (segment (start 59.256 82.776) (end 59.256 88.044) (width 2) (layer B.Cu) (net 6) (status 10))
 (segment (start 59.256 103.284) (end 55.14 107.4) (width 2) (layer B.Cu) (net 6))
 (segment (start 59.256 88.044) (end 59.256 103.284) (width 2) (layer B.Cu) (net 6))
 (segment (start 26.744 98.016) (end 26.744 78.472) (width 2) (layer B.Cu) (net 6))
 (segment (start 36.904 108.176) (end 26.744 98.016) (width 2) (layer B.Cu) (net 6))
 (segment (start 55.192 107.16) (end 54.176 108.176) (width 2) (layer B.Cu) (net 6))
 (segment (start 54.176 108.176) (end 36.904 108.176) (width 2) (layer B.Cu) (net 6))
 (segment (start 50.06 112.48) (end 41.932 112.48) (width 2) (layer B.Cu) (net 7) (status 30))
 (segment (start 33.804 112.48) (end 36.852 112.48) (width 2) (layer B.Cu) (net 8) (status 20))
 (segment (start 21.612 100.288) (end 33.804 112.48) (width 2) (layer B.Cu) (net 8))
 (segment (start 22.012 73.472) (end 21.664 73.124) (width 2) (layer B.Cu) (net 8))
 (segment (start 26.744 73.472) (end 22.012 73.472) (width 2) (layer B.Cu) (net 8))
 (segment (start 21.664 73.124) (end 21.612 100.288) (width 2) (layer B.Cu) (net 8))
 (segment (start 21.612 56.412) (end 25.704 52.32) (width 2) (layer B.Cu) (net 8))
 (segment (start 25.704 52.32) (end 26.6 52.32) (width 2) (layer B.Cu) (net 8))
 (segment (start 21.664 73.124) (end 21.612 61.172) (width 2) (layer B.Cu) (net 8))
 (segment (start 21.612 61.172) (end 21.612 56.412) (width 2) (layer B.Cu) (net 8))
 (segment (start 34.644 42.872) (end 34.788 42.872) (width 2) (layer B.Cu) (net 8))
 (segment (start 26.576 50.94) (end 34.644 42.872) (width 2) (layer B.Cu) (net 8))
 (segment (start 26.6 52.32) (end 26.576 52.296) (width 2) (layer B.Cu) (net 8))
 (segment (start 26.576 52.296) (end 26.576 50.94) (width 2) (layer B.Cu) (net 8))
 (segment (start 36.852 40.808) (end 34.788 42.872) (width 2) (layer B.Cu) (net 8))
 (segment (start 36.852 31.2) (end 36.852 40.808) (width 2) (layer B.Cu) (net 8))
 (segment (start 41.456 42.872) (end 34.788 42.872) (width 2) (layer B.Cu) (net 8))
 (segment (start 41.656 42.672) (end 41.456 42.872) (width 2) (layer B.Cu) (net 8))
 (segment (start 41.932 31.2) (end 50.06 31.2) (width 2) (layer B.Cu) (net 1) (status 30))
 (segment (start 62.812 99.032) (end 62.812 96.492) (width 2) (layer B.Cu) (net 9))
 (segment (start 62.812 96.492) (end 62.812 92.936) (width 2) (layer B.Cu) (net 9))
 (segment (start 69.2 85.024) (end 69.2 81.764) (width 2) (layer B.Cu) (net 9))
 (segment (start 62.812 92.936) (end 62.812 91.412) (width 2) (layer B.Cu) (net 9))
 (segment (start 62.812 91.412) (end 69.2 85.024) (width 2) (layer B.Cu) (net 9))
 (segment (start 63.066 58.392) (end 63.066 61.44) (width 2) (layer B.Cu) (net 11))
 (segment (start 63.066 63.98) (end 63.066 61.44) (width 2) (layer B.Cu) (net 11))
 (segment (start 63.066 63.98) (end 63.066 68.806) (width 2) (layer B.Cu) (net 11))
 (segment (start 67.134 72.874) (end 69.2 72.874) (width 2) (layer B.Cu) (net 11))
 (segment (start 63.066 68.806) (end 67.134 72.874) (width 2) (layer B.Cu) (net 11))
 (segment (start 72.464 43.66) (end 70.432 41.628) (width 1) (layer B.Cu) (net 15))
 (segment (start 72.464 49.756) (end 72.464 43.66) (width 1) (layer B.Cu) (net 15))
 (segment (start 70.432 41.628) (end 70.432 40.104) (width 1) (layer B.Cu) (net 15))
 (segment (start 67.892 51.28) (end 70.94 51.28) (width 1) (layer B.Cu) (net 15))
 (segment (start 70.94 51.28) (end 72.464 49.756) (width 1) (layer B.Cu) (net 15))
 (segment (start 69.416 48.74) (end 67.892 48.74) (width 1) (layer B.Cu) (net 16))
 (segment (start 70.432 47.724) (end 69.416 48.74) (width 1) (layer B.Cu) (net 16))
 (segment (start 70.432 44.676) (end 70.432 47.724) (width 1) (layer B.Cu) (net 16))
 (segment (start 67.892 40.104) (end 67.892 42.136) (width 1) (layer B.Cu) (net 16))
 (segment (start 67.892 42.136) (end 70.432 44.676) (width 1) (layer B.Cu) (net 16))
 (segment (start 34.312 85.368) (end 34.312 85.57) (width 2) (layer B.Cu) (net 17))
 (segment (start 34.312 63.668) (end 34.788 63.192) (width 2) (layer B.Cu) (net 17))
 (segment (start 34.312 85.57) (end 34.312 63.668) (width 2) (layer B.Cu) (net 17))
 (segment (start 26.6 57.4) (end 31.34 57.4) (width 2) (layer B.Cu) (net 17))
 (segment (start 34.788 60.848) (end 34.788 63.192) (width 2) (layer B.Cu) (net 17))
 (segment (start 31.34 57.4) (end 34.788 60.848) (width 2) (layer B.Cu) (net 17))
 (segment (start 41.392 63.192) (end 34.788 63.192) (width 2) (layer B.Cu) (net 17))
 (segment (start 71.706 75.414) (end 71.956 75.664) (width 2) (layer B.Cu) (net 3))
 (segment (start 69.2 75.414) (end 71.706 75.414) (width 2) (layer B.Cu) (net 3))
 (segment (start 67.892 53.82) (end 67.892 62.456) (width 1) (layer B.Cu) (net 3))
 (segment (start 72.824 75.664) (end 71.956 75.664) (width 2) (layer B.Cu) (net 3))
 (segment (start 74.52 77.36) (end 72.824 75.664) (width 2) (layer B.Cu) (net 3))
 (segment (start 72.6 76.308) (end 71.956 75.664) (width 2) (layer B.Cu) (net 3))
 (segment (start 72.6 102.216) (end 72.6 76.308) (width 2) (layer B.Cu) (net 3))
 (segment (start 84.148 103.604) (end 73.988 103.604) (width 2) (layer B.Cu) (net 3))
 (segment (start 73.988 103.604) (end 72.6 102.216) (width 2) (layer B.Cu) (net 3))
 (segment (start 67.892 67.152) (end 67.892 62.456) (width 2) (layer B.Cu) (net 3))
 (segment (start 71.956 75.664) (end 71.956 71.216) (width 2) (layer B.Cu) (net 3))
 (segment (start 71.956 71.216) (end 67.892 67.152) (width 2) (layer B.Cu) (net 3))
 (segment (start 73.56 104.032) (end 73.988 103.604) (width 1) (layer B.Cu) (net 3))
 (segment (start 73.56 108.36) (end 73.56 104.032) (width 1) (layer B.Cu) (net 3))
 (segment (start 59.256 52.484) (end 57.68 54.06) (width 2) (layer B.Cu) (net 13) (status 20))
 (segment (start 59.256 47.216) (end 59.256 52.484) (width 2) (layer B.Cu) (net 13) (status 10))
 (segment (start 59.256 72.616) (end 65.86 79.22) (width 2) (layer B.Cu) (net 13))
 (segment (start 65.864 79.224) (end 65.86 79.22) (width 2) (layer B.Cu) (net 13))
 (segment (start 69.2 79.224) (end 65.864 79.224) (width 2) (layer B.Cu) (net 13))
 (segment (start 63.1 85.028) (end 62.812 85.316) (width 2) (layer B.Cu) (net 13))
 (segment (start 65.86 79.22) (end 63.1 81.98) (width 2) (layer B.Cu) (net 13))
 (segment (start 63.1 81.98) (end 63.1 85.028) (width 2) (layer B.Cu) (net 13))
 (segment (start 59.256 72.616) (end 59.256 52.484) (width 2) (layer B.Cu) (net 13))
 (segment (start 59.256 72.616) (end 59.256 75.704) (width 2) (layer B.Cu) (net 13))
 (segment (start 55.1 79.86) (end 55.1 81.36) (width 2) (layer B.Cu) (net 13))
 (segment (start 59.256 75.704) (end 55.1 79.86) (width 2) (layer B.Cu) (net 13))
 (segment (start 55.14 87.08) (end 55.1 81.36) (width 2) (layer B.Cu) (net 13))
 (segment (start 34.312 98.27) (end 39.19 98.27) (width 2) (layer B.Cu) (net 13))
 (segment (start 50.38 87.08) (end 55.14 87.08) (width 2) (layer B.Cu) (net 13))
 (segment (start 39.19 98.27) (end 50.38 87.08) (width 2) (layer B.Cu) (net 13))
 (segment (start 89.228 90.904) (end 88.212 89.888) (width 2) (layer B.Cu) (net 4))
 (segment (start 90.244 102.08) (end 90.244 91.92) (width 2) (layer B.Cu) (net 4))
 (segment (start 86.688 103.604) (end 88.72 103.604) (width 2) (layer B.Cu) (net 4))
 (segment (start 90.244 91.92) (end 89.228 90.904) (width 2) (layer B.Cu) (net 4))
 (segment (start 88.72 103.604) (end 90.244 102.08) (width 2) (layer B.Cu) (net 4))
 (segment (start 86.688 91.412) (end 86.688 93.952) (width 2) (layer B.Cu) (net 4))
 (segment (start 88.212 89.888) (end 86.688 91.412) (width 2) (layer B.Cu) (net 4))
 (segment (start 88.212 86.68) (end 88.212 89.888) (width 2) (layer B.Cu) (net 4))
 (segment (start 79.6 77.36) (end 79.6 78.068) (width 2) (layer B.Cu) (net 4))
 (segment (start 79.6 78.068) (end 88.212 86.68) (width 2) (layer B.Cu) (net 4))
 (segment (start 77.72 108.36) (end 78.6 107.48) (width 1) (layer B.Cu) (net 18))
 (segment (start 76.1 108.36) (end 77.72 108.36) (width 1) (layer B.Cu) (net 18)))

